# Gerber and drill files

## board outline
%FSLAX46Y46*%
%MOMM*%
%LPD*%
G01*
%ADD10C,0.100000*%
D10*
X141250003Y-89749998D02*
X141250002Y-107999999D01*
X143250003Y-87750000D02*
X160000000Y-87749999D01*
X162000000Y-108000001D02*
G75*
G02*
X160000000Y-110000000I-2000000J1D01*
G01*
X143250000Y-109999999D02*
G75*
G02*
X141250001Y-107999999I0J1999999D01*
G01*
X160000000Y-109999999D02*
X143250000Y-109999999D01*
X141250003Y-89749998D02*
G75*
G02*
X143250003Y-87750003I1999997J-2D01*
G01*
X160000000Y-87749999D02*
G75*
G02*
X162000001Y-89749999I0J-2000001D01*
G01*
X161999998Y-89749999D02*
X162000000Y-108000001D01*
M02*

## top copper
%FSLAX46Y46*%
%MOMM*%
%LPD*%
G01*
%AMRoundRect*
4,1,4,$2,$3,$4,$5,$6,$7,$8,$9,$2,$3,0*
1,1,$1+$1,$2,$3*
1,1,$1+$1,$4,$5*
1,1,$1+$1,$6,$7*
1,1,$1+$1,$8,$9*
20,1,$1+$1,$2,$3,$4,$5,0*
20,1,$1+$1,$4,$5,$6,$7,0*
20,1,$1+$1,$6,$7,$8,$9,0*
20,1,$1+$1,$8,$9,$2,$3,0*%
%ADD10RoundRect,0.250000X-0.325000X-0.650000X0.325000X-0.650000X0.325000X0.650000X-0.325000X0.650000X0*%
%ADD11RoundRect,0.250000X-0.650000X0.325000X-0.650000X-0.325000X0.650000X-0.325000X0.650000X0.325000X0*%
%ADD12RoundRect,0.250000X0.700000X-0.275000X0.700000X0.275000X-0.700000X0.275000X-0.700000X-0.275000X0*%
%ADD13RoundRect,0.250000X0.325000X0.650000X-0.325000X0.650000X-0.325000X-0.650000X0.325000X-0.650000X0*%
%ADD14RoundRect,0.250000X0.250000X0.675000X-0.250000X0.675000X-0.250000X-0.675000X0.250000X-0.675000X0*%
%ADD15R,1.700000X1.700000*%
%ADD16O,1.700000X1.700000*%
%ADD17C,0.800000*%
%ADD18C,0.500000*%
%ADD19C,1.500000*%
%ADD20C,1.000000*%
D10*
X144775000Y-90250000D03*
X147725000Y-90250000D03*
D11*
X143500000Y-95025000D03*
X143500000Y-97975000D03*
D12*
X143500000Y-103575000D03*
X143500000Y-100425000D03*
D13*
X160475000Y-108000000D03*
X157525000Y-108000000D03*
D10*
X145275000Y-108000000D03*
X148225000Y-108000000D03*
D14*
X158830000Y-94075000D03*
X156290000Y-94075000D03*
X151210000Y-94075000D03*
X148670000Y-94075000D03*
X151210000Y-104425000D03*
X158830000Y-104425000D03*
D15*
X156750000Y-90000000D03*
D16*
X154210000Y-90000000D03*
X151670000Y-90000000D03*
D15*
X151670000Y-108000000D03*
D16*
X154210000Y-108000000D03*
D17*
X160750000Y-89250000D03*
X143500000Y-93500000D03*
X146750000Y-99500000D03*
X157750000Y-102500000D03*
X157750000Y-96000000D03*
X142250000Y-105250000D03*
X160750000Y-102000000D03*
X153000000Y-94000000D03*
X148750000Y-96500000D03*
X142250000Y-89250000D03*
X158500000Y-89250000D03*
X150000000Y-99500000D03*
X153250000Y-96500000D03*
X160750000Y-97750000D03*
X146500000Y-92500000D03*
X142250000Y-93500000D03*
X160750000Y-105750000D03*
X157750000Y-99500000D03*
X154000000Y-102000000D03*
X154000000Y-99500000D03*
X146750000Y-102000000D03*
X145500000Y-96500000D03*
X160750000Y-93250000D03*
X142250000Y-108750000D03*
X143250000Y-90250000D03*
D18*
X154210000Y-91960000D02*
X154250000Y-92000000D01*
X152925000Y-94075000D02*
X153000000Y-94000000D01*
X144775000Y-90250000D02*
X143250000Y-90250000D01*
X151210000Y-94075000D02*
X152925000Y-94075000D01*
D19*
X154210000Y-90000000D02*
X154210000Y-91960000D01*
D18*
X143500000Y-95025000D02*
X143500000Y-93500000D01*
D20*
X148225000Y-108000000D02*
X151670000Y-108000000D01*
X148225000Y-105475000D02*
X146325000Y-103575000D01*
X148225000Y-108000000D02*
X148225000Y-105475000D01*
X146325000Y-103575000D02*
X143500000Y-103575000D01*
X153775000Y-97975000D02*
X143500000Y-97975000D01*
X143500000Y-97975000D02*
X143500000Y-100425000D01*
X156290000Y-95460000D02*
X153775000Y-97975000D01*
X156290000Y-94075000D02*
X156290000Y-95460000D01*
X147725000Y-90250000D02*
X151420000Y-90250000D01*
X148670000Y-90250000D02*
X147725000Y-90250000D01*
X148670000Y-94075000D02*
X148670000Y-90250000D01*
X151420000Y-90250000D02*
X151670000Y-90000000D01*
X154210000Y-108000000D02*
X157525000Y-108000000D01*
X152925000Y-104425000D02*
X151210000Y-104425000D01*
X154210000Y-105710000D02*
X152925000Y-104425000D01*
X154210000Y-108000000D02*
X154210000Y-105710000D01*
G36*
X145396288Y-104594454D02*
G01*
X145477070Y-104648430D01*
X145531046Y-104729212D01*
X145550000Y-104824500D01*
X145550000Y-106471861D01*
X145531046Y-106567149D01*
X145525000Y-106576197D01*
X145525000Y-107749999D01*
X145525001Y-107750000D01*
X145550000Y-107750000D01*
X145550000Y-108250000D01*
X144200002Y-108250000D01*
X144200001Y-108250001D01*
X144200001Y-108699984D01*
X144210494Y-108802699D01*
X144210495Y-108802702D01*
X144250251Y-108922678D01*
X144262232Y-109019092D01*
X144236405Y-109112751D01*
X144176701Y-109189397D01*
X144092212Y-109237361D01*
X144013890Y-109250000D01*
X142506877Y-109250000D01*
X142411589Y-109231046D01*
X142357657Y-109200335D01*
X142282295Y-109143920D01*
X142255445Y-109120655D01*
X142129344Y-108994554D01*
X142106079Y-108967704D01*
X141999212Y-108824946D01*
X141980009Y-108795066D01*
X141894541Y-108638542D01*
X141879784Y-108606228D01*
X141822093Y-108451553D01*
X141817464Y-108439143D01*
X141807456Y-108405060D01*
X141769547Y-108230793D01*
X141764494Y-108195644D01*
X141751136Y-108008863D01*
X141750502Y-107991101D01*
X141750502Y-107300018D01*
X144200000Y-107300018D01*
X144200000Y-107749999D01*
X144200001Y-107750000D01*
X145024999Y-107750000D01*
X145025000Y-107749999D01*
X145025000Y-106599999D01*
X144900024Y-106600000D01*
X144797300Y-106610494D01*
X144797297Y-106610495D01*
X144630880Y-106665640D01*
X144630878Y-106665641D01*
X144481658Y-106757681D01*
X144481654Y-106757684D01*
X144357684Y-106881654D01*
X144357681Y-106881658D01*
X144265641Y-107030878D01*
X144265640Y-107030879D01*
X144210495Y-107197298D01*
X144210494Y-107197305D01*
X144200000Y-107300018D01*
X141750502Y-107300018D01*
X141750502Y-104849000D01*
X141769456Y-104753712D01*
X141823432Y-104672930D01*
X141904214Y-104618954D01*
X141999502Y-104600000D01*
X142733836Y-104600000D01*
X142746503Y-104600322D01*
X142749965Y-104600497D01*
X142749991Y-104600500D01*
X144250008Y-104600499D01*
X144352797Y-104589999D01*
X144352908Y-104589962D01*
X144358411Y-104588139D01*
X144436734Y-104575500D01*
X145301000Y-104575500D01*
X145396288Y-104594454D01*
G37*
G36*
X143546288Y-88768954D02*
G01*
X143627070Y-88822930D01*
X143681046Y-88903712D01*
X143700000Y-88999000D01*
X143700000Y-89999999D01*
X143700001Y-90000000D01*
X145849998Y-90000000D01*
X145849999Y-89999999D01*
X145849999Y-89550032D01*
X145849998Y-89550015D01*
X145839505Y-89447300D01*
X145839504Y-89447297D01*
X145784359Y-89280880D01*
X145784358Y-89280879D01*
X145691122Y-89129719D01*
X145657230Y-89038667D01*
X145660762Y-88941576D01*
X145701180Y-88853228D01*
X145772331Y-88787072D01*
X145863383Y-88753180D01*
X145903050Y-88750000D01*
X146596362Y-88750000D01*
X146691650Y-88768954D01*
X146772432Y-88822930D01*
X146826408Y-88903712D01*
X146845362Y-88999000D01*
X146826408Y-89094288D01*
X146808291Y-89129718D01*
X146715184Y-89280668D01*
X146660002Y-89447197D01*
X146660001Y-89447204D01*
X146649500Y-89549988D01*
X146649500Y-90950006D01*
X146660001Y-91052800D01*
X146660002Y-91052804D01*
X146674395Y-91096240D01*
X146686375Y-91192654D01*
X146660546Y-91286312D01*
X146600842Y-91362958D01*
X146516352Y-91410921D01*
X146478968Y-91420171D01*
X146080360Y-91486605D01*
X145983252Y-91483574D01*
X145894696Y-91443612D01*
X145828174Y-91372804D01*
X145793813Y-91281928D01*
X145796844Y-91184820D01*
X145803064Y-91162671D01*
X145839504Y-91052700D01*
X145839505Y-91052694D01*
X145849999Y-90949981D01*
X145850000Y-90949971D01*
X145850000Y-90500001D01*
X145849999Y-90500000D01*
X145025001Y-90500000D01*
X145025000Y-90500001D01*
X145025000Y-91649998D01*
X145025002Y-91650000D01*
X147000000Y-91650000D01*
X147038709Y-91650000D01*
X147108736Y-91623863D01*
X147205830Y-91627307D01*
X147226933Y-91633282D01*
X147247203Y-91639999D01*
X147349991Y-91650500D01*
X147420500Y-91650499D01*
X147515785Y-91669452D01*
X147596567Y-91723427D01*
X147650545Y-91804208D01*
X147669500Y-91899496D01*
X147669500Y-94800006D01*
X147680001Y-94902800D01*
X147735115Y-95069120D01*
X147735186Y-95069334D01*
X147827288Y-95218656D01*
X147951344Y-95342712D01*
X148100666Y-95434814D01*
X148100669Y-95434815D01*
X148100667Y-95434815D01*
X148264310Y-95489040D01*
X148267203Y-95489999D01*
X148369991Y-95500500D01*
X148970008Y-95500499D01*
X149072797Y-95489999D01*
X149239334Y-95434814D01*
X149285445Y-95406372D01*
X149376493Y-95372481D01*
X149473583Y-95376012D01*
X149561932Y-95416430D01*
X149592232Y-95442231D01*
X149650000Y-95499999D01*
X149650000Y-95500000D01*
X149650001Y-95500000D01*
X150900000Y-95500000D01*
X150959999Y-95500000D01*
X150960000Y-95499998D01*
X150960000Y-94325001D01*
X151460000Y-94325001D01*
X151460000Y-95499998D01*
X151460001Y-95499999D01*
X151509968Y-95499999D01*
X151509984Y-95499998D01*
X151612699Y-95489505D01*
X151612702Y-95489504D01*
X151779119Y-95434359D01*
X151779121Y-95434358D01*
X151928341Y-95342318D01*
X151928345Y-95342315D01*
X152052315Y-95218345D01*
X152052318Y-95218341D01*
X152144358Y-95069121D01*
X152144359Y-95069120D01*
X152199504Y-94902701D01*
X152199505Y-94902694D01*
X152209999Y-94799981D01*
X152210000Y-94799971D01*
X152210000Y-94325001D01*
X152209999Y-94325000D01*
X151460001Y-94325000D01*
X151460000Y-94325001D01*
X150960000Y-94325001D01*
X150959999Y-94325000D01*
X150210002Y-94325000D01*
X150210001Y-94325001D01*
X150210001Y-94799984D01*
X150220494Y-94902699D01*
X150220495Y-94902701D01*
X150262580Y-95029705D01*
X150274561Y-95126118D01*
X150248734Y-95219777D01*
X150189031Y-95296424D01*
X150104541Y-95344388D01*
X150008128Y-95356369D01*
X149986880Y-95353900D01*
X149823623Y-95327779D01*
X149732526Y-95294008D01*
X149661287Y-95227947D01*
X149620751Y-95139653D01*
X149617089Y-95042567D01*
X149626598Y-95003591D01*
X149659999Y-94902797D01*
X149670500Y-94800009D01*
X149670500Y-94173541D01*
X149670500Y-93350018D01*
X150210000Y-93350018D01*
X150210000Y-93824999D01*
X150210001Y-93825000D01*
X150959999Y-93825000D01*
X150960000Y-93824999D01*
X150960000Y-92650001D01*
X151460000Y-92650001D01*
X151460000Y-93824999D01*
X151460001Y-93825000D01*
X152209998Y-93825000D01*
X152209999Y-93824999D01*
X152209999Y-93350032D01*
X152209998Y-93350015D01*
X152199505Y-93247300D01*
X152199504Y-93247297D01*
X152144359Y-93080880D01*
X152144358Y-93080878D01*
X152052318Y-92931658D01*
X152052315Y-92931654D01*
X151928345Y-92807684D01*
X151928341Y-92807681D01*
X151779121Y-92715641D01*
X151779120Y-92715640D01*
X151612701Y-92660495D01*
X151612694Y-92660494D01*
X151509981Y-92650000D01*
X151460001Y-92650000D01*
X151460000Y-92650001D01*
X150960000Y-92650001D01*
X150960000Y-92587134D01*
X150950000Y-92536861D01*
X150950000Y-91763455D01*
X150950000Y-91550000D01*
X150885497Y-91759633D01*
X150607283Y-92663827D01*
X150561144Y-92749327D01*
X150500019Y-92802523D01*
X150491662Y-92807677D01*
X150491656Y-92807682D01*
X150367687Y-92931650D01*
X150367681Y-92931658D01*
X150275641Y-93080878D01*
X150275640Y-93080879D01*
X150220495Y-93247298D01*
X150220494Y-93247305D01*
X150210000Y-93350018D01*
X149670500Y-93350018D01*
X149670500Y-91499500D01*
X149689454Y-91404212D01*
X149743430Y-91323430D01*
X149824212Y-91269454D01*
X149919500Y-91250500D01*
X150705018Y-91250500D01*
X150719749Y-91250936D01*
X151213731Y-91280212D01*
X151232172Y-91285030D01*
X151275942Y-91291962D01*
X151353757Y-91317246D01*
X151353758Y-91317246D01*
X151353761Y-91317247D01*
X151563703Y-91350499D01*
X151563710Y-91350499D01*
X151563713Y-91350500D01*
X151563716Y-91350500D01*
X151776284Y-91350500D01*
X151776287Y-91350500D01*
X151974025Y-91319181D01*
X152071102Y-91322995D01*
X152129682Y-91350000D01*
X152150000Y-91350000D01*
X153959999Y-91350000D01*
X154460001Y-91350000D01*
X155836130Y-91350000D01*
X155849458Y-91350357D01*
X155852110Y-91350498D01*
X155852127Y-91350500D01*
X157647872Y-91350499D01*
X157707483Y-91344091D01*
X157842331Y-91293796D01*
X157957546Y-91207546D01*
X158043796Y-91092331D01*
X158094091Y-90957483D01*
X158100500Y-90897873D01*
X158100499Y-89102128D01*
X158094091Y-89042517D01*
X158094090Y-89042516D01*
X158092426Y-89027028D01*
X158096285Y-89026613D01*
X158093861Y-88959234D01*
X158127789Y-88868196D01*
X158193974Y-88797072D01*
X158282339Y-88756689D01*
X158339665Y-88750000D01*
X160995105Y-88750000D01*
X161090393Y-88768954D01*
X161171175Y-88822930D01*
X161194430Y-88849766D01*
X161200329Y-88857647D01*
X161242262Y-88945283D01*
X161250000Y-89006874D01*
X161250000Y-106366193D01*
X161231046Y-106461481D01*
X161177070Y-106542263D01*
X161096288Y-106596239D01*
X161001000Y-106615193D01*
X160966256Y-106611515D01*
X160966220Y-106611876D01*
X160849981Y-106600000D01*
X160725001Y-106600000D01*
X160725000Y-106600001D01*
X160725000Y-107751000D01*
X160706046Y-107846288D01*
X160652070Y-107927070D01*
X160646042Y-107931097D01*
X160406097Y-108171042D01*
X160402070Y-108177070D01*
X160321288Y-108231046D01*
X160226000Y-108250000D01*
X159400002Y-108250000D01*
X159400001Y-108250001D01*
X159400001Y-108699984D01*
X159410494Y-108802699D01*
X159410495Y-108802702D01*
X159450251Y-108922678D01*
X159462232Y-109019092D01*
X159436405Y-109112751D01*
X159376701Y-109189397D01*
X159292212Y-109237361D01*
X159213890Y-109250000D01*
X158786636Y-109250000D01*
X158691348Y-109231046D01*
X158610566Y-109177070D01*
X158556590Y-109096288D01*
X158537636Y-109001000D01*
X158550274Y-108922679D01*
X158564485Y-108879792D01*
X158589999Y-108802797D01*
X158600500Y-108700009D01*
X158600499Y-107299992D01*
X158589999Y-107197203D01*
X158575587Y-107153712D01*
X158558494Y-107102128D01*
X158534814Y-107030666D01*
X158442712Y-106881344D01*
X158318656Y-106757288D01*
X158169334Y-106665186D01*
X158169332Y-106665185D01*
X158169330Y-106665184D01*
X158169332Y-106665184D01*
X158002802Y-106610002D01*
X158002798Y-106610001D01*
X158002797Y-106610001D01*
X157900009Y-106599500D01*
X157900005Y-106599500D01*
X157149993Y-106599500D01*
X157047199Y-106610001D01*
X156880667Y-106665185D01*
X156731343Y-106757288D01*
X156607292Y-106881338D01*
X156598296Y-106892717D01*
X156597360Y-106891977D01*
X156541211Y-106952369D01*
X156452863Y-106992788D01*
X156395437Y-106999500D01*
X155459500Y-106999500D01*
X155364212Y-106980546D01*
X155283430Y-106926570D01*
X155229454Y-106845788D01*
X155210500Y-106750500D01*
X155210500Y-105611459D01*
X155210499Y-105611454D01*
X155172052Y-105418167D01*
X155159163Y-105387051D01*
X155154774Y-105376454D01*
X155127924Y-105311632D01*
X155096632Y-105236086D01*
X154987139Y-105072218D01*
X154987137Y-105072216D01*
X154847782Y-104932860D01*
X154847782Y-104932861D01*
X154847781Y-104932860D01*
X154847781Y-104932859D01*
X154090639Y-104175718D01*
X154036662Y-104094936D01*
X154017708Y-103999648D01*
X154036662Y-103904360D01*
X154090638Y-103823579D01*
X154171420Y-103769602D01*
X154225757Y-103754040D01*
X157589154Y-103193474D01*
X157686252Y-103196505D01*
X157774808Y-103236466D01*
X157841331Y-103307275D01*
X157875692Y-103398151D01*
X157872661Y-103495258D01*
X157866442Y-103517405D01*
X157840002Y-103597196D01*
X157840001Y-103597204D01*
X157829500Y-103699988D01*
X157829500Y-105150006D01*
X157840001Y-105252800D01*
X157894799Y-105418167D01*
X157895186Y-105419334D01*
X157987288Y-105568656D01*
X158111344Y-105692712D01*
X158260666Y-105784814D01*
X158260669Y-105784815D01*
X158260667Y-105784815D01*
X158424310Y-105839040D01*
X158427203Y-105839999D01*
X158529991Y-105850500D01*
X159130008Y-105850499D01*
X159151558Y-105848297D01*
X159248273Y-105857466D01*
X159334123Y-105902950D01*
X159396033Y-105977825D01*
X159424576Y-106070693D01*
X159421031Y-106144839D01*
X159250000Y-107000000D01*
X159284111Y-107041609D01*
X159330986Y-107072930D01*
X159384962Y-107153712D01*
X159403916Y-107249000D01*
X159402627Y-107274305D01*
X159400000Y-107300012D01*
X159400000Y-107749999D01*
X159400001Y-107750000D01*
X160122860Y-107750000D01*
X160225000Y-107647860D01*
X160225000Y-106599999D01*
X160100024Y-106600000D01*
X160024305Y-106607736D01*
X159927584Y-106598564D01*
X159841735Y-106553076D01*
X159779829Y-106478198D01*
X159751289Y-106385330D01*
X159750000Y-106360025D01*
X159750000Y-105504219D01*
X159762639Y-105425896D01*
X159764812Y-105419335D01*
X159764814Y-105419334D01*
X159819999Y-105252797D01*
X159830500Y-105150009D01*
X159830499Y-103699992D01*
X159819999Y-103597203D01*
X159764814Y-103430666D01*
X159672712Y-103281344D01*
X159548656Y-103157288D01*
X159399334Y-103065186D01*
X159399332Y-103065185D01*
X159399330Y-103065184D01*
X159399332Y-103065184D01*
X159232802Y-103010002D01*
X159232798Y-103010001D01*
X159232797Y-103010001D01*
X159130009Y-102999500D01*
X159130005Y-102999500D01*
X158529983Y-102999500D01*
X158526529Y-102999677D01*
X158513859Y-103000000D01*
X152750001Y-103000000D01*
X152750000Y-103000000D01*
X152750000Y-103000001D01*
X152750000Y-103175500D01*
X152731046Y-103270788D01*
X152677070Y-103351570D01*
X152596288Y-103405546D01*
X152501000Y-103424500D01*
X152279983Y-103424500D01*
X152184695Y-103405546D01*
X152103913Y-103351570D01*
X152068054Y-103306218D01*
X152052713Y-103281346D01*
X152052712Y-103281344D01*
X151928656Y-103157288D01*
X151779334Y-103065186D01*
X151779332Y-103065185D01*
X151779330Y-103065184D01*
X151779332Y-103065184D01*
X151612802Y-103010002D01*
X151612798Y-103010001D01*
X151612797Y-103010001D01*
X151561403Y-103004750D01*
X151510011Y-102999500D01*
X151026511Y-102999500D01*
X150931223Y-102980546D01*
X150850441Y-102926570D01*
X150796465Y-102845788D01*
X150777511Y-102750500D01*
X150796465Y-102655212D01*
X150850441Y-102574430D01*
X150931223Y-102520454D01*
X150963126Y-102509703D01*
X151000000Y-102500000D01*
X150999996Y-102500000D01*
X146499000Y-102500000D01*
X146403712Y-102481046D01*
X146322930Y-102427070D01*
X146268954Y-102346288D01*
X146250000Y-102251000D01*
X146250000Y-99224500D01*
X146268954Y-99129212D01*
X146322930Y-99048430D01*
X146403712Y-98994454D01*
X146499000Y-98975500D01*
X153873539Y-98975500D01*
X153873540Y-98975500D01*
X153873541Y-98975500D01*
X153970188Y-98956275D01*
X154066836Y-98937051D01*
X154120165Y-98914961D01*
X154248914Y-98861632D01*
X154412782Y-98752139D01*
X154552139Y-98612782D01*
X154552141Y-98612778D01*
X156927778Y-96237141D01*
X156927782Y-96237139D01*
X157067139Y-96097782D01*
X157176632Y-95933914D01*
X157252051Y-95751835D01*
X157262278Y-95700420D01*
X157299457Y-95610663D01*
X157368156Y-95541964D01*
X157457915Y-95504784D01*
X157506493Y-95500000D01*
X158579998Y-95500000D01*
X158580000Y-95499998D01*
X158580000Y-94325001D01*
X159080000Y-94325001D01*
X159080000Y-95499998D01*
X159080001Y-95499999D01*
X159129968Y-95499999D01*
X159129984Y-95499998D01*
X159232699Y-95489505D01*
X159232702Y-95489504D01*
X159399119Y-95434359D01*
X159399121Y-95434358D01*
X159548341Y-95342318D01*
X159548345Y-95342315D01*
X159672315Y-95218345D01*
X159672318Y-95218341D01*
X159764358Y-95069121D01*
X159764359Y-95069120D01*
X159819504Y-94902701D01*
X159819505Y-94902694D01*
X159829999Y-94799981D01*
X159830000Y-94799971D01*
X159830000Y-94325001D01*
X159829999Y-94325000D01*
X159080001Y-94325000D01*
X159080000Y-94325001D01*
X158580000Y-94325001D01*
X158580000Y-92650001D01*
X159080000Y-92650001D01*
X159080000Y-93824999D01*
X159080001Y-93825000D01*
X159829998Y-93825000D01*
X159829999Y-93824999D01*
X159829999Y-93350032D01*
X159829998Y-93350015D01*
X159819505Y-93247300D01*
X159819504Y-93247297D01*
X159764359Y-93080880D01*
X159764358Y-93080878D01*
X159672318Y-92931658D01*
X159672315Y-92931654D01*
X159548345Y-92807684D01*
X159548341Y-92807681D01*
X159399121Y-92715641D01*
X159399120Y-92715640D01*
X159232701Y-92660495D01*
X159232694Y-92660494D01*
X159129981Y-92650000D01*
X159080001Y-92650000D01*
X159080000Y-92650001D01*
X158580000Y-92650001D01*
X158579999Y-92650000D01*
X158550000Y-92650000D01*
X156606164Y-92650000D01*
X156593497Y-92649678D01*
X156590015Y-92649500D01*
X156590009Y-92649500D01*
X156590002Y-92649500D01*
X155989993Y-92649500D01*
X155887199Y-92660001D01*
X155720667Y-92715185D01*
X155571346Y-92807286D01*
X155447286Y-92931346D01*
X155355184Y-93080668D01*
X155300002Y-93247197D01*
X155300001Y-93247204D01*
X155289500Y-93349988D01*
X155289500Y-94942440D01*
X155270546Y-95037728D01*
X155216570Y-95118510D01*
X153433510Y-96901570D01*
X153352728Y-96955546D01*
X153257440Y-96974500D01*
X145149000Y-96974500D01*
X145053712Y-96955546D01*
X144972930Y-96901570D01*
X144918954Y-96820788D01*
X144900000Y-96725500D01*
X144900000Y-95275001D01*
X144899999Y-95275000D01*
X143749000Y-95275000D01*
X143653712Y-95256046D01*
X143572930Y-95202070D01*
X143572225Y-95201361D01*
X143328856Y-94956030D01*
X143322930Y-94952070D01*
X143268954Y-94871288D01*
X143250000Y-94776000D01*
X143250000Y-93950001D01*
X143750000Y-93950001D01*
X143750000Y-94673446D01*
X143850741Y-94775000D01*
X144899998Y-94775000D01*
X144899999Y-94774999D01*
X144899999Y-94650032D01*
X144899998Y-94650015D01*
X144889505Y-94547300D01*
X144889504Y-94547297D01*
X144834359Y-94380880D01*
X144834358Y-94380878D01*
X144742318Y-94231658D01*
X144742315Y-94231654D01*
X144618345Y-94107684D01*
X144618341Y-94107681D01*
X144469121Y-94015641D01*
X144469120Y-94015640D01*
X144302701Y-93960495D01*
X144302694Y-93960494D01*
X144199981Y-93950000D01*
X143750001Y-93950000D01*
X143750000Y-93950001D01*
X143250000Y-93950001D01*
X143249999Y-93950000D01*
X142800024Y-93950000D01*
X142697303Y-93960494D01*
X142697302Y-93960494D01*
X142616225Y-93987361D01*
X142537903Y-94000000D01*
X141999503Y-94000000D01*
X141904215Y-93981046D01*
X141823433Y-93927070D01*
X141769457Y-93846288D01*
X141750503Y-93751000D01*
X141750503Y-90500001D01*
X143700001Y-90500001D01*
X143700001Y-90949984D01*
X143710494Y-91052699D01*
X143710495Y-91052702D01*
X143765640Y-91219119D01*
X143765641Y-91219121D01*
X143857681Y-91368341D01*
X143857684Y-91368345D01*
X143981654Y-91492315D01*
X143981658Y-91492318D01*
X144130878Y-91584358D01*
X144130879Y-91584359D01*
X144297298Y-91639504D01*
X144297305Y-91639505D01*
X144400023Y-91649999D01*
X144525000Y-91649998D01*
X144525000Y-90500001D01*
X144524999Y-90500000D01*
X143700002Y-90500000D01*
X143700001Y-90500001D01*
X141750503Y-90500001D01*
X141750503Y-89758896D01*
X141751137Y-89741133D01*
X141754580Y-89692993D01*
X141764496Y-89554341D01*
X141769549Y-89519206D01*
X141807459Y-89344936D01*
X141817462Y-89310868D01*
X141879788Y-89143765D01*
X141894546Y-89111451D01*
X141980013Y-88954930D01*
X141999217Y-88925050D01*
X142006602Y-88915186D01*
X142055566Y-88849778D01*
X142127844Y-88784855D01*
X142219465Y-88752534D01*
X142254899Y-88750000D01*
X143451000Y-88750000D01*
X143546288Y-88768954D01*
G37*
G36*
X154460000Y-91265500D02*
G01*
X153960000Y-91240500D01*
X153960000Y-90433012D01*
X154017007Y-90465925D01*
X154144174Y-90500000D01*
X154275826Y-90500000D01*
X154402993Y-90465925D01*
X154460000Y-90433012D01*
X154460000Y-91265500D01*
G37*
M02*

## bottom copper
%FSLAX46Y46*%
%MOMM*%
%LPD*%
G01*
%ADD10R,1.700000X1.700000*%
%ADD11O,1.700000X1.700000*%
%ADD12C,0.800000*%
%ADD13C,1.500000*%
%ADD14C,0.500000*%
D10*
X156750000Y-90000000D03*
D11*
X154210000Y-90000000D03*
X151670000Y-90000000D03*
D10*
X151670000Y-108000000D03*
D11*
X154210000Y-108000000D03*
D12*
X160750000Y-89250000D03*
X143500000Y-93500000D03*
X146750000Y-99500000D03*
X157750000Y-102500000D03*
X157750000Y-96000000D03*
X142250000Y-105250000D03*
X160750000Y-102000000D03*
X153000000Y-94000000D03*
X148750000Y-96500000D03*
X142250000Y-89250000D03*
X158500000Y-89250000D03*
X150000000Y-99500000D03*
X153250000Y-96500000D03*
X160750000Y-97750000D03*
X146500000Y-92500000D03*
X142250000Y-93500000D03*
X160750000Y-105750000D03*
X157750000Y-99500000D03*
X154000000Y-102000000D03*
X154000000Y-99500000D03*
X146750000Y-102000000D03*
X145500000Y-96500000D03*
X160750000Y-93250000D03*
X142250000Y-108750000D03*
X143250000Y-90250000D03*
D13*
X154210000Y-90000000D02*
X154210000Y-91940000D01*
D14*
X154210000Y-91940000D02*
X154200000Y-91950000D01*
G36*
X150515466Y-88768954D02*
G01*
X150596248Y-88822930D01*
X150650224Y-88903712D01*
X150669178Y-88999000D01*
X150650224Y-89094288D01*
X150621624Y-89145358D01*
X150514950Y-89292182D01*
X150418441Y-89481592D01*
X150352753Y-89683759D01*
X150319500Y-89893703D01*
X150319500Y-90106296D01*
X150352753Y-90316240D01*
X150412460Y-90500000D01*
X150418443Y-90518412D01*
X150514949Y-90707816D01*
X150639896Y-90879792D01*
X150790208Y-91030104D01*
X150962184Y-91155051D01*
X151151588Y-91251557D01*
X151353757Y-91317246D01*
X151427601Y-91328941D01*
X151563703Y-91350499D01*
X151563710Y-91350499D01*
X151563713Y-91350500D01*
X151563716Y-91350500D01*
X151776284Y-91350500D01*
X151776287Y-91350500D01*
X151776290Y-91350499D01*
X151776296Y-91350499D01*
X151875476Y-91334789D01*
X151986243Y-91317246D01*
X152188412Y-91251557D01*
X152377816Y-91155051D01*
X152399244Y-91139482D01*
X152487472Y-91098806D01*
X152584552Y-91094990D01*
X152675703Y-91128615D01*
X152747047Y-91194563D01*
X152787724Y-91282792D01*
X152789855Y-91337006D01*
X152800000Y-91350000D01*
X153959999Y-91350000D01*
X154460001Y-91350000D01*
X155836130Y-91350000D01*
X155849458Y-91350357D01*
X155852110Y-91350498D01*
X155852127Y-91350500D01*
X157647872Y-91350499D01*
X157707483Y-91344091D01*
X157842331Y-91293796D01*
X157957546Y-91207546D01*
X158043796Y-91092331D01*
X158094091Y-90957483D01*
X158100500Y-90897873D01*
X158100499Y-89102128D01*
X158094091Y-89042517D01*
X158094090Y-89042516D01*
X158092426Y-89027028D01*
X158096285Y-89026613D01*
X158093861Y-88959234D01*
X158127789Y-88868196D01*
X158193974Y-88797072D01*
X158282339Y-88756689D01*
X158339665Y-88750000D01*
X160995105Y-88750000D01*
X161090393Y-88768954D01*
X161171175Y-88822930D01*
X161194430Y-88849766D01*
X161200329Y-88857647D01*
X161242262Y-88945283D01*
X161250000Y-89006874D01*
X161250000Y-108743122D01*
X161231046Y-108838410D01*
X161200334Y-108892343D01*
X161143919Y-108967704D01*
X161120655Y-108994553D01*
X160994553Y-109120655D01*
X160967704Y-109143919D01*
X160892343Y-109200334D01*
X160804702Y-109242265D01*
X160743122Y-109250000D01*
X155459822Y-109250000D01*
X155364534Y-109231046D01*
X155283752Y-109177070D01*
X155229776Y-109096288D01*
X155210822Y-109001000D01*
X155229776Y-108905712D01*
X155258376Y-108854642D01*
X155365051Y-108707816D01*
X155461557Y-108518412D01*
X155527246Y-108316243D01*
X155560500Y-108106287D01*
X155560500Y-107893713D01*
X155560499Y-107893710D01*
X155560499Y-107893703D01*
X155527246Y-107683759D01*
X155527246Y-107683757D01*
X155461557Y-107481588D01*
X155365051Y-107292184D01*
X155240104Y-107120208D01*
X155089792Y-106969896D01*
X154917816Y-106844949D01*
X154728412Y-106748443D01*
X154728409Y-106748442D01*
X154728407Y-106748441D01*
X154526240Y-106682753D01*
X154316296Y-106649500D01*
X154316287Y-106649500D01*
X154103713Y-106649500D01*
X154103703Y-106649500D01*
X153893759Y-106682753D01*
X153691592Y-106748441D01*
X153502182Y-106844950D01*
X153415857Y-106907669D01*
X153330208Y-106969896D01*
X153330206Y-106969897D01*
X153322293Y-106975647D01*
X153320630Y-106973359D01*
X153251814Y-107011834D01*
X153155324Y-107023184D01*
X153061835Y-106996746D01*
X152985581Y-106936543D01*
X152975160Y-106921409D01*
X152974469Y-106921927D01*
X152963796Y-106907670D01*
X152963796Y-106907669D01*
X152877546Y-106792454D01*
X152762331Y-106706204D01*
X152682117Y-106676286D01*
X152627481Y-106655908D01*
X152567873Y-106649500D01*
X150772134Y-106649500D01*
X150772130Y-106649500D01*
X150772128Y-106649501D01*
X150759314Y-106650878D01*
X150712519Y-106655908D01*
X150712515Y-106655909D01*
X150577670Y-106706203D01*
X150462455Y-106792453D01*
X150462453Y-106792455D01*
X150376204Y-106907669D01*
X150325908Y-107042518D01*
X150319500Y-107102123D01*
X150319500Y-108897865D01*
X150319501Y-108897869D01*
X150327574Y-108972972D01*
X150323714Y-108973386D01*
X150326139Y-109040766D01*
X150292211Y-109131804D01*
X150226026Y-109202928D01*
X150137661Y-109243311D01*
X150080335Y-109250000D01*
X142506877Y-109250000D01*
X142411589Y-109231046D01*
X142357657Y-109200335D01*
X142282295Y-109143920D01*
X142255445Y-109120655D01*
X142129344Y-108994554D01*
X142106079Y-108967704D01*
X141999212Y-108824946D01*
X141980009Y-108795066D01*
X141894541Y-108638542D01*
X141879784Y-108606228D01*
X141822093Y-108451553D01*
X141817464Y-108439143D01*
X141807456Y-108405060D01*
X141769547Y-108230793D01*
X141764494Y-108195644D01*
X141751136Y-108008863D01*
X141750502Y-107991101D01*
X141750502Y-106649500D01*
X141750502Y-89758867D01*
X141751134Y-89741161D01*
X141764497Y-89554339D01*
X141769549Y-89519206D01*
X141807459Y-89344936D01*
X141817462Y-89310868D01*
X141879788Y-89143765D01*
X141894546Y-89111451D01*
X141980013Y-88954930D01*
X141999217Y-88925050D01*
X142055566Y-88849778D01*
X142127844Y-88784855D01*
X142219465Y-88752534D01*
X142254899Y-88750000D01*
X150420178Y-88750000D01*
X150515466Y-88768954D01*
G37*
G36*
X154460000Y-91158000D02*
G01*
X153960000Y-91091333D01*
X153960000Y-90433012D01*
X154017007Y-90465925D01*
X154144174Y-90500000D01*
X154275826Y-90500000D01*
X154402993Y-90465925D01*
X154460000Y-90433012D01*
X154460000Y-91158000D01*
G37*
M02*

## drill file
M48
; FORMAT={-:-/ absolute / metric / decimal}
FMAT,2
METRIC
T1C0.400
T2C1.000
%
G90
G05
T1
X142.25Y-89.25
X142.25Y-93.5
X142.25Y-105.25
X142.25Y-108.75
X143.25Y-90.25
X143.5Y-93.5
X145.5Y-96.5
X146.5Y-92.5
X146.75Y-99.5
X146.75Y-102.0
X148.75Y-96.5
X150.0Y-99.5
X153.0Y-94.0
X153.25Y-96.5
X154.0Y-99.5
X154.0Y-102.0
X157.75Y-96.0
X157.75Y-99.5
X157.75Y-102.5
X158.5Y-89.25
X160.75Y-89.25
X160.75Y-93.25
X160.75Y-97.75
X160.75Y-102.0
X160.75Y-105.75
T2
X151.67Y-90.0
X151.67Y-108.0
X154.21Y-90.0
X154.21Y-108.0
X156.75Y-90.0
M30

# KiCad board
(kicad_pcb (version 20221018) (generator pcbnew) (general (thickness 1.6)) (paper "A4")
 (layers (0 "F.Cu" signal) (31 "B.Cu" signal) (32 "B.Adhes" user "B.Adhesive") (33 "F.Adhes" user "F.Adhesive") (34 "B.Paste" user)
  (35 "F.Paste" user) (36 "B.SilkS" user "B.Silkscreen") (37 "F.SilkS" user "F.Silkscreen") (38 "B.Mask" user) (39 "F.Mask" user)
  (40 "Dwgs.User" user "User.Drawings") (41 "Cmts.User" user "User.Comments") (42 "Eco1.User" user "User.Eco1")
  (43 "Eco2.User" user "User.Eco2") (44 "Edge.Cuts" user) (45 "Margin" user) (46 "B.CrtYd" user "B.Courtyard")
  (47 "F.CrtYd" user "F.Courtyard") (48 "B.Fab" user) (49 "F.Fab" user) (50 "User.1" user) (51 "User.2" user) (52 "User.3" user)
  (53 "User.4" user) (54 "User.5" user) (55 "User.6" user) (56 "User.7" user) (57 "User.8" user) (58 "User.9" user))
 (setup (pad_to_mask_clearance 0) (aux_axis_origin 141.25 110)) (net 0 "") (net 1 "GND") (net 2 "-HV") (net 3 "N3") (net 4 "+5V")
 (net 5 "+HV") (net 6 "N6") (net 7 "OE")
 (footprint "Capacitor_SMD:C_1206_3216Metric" (layer "F.Cu") (at 146.25 90.25)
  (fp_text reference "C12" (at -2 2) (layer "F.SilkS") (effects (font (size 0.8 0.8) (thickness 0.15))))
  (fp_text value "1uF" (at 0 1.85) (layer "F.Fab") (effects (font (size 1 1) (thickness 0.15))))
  (pad "1" smd roundrect (at -1.475 0) (size 1.15 1.8) (layers "F.Cu" "F.Paste" "F.Mask") (roundrect_rratio 0.2173913043) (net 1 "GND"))
  (pad "2" smd roundrect (at 1.475 0) (size 1.15 1.8) (layers "F.Cu" "F.Paste" "F.Mask") (roundrect_rratio 0.2173913043) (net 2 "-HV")))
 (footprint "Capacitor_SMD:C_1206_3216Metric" (layer "F.Cu") (at 143.5 96.5 -90)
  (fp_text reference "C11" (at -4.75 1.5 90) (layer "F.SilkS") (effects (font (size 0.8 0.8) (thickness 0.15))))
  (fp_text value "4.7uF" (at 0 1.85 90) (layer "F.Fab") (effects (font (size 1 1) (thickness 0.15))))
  (pad "1" smd roundrect (at -1.475 0 270) (size 1.15 1.8) (layers "F.Cu" "F.Paste" "F.Mask") (roundrect_rratio 0.2173913043) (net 1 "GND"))
  (pad "2" smd roundrect (at 1.475 0 270) (size 1.15 1.8) (layers "F.Cu" "F.Paste" "F.Mask") (roundrect_rratio 0.2173913043) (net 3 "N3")))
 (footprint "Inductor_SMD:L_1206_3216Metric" (layer "F.Cu") (at 143.5 102 90)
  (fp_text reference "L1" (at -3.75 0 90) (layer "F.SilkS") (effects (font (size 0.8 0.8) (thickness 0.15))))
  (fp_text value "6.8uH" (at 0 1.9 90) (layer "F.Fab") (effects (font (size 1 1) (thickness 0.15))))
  (pad "1" smd roundrect (at -1.575 0 90) (size 1.05 1.9) (layers "F.Cu" "F.Paste" "F.Mask") (roundrect_rratio 0.2380952381) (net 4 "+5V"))
  (pad "2" smd roundrect (at 1.575 0 90) (size 1.05 1.9) (layers "F.Cu" "F.Paste" "F.Mask") (roundrect_rratio 0.2380952381) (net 3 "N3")))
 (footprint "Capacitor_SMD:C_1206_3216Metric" (layer "F.Cu") (at 159 108 180)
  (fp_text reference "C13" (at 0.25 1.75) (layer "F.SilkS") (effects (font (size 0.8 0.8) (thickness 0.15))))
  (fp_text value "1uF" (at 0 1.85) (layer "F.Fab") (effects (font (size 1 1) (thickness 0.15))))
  (pad "1" smd roundrect (at -1.475 0 180) (size 1.15 1.8) (layers "F.Cu" "F.Paste" "F.Mask") (roundrect_rratio 0.2173913043) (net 1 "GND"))
  (pad "2" smd roundrect (at 1.475 0 180) (size 1.15 1.8) (layers "F.Cu" "F.Paste" "F.Mask") (roundrect_rratio 0.2173913043) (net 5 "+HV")))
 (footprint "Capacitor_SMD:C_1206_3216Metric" (layer "F.Cu") (at 146.75 108)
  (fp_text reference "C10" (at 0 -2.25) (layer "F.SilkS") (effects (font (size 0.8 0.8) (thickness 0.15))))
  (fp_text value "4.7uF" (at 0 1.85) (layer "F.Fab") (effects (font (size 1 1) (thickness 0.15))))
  (pad "1" smd roundrect (at -1.475 0) (size 1.15 1.8) (layers "F.Cu" "F.Paste" "F.Mask") (roundrect_rratio 0.2173913043) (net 1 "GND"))
  (pad "2" smd roundrect (at 1.475 0) (size 1.15 1.8) (layers "F.Cu" "F.Paste" "F.Mask") (roundrect_rratio 0.2173913043) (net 4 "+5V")))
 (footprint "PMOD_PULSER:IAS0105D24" (layer "F.Cu") (at 153.75 99.25 180)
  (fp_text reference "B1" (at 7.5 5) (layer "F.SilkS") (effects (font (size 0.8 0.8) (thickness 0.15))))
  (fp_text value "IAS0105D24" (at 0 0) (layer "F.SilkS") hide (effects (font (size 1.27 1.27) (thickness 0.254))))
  (pad "1" smd roundrect (at -5.08 5.175 180) (size 1 1.85) (layers "F.Cu" "F.Paste" "F.Mask") (roundrect_rratio 0.25) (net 1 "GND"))
  (pad "2" smd roundrect (at -2.54 5.175 180) (size 1 1.85) (layers "F.Cu" "F.Paste" "F.Mask") (roundrect_rratio 0.25) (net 3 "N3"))
  (pad "4" smd roundrect (at 2.54 5.175 180) (size 1 1.85) (layers "F.Cu" "F.Paste" "F.Mask") (roundrect_rratio 0.25) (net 1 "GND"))
  (pad "5" smd roundrect (at 5.08 5.175 180) (size 1 1.85) (layers "F.Cu" "F.Paste" "F.Mask") (roundrect_rratio 0.25) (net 2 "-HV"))
  (pad "7" smd roundrect (at 2.54 -5.175 180) (size 1 1.85) (layers "F.Cu" "F.Paste" "F.Mask") (roundrect_rratio 0.25) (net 5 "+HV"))
  (pad "10" smd roundrect (at -5.08 -5.175 180) (size 1 1.85) (layers "F.Cu" "F.Paste" "F.Mask") (roundrect_rratio 0.25) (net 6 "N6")))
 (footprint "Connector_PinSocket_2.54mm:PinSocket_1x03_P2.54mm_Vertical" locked (layer "B.Cu") (at 156.75 90 90)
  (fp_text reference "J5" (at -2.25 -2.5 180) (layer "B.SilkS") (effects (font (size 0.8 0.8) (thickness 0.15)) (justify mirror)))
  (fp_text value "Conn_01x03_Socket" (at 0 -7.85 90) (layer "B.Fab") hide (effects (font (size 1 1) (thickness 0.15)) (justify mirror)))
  (pad "1" thru_hole rect locked (at 0 0 90) (size 1.7 1.7) (drill 1) (layers "*.Cu" "*.Mask") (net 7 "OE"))
  (pad "2" thru_hole oval locked (at 0 -2.54 90) (size 1.7 1.7) (drill 1) (layers "*.Cu" "*.Mask") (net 1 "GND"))
  (pad "3" thru_hole oval locked (at 0 -5.08 90) (size 1.7 1.7) (drill 1) (layers "*.Cu" "*.Mask") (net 2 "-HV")))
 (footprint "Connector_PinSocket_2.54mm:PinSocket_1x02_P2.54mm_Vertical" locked (layer "B.Cu") (at 151.67 108 -90)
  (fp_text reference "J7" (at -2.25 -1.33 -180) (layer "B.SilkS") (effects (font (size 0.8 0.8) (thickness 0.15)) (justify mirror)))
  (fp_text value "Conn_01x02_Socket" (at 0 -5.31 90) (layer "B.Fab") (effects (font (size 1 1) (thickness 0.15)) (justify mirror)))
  (pad "1" thru_hole rect locked (at 0 0 270) (size 1.7 1.7) (drill 1) (layers "*.Cu" "*.Mask") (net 4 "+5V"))
  (pad "2" thru_hole oval locked (at 0 -2.54 270) (size 1.7 1.7) (drill 1) (layers "*.Cu" "*.Mask") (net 5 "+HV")))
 (gr_line (start 141.250003 89.749998) (end 141.250002 107.999999) (stroke (width 0.1) (type default)) (layer "Edge.Cuts"))
 (gr_line (start 143.250003 87.75) (end 160 87.749999) (stroke (width 0.1) (type default)) (layer "Edge.Cuts"))
 (gr_arc (start 162 108.000001) (mid 161.414213 109.414213) (end 160 109.999999) (stroke (width 0.1) (type default)) (layer "Edge.Cuts"))
 (gr_arc (start 143.25 109.999999) (mid 141.835786 109.414213) (end 141.250002 107.999999) (stroke (width 0.1) (type default))
  (layer "Edge.Cuts"))
 (gr_line (start 160 109.999999) (end 143.25 109.999999) (stroke (width 0.1) (type default)) (layer "Edge.Cuts"))
 (gr_arc (start 141.250003 89.749998) (mid 141.83579 88.335786) (end 143.250003 87.75) (stroke (width 0.1) (type default))
  (layer "Edge.Cuts"))
 (gr_arc (start 160 87.749999) (mid 161.414214 88.335785) (end 161.999998 89.749999) (stroke (width 0.1) (type default)) (layer "Edge.Cuts"))
 (gr_line (start 161.999998 89.749999) (end 162 108.000001) (stroke (width 0.1) (type default)) (layer "Edge.Cuts"))
 (segment (start 154.21 91.96) (end 154.25 92) (width 0.5) (layer "F.Cu") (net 1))
 (segment (start 152.925 94.075) (end 153 94) (width 0.5) (layer "F.Cu") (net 1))
 (segment (start 144.775 90.25) (end 143.25 90.25) (width 0.5) (layer "F.Cu") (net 1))
 (segment (start 151.21 94.075) (end 152.925 94.075) (width 0.5) (layer "F.Cu") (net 1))
 (segment (start 154.21 90) (end 154.21 91.96) (width 1.5) (layer "F.Cu") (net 1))
 (segment (start 143.5 95.025) (end 143.5 93.5) (width 0.5) (layer "F.Cu") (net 1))
 (via (at 160.75 89.25) (size 0.8) (drill 0.4) (layers "F.Cu" "B.Cu") (free) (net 1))
 (via (at 143.5 93.5) (size 0.8) (drill 0.4) (layers "F.Cu" "B.Cu") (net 1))
 (via (at 146.75 99.5) (size 0.8) (drill 0.4) (layers "F.Cu" "B.Cu") (free) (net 1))
 (via (at 157.75 102.5) (size 0.8) (drill 0.4) (layers "F.Cu" "B.Cu") (free) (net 1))
 (via (at 157.75 96) (size 0.8) (drill 0.4) (layers "F.Cu" "B.Cu") (free) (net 1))
 (via (at 142.25 105.25) (size 0.8) (drill 0.4) (layers "F.Cu" "B.Cu") (free) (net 1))
 (via (at 160.75 102) (size 0.8) (drill 0.4) (layers "F.Cu" "B.Cu") (free) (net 1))
 (via (at 153 94) (size 0.8) (drill 0.4) (layers "F.Cu" "B.Cu") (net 1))
 (via (at 148.75 96.5) (size 0.8) (drill 0.4) (layers "F.Cu" "B.Cu") (free) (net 1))
 (via (at 142.25 89.25) (size 0.8) (drill 0.4) (layers "F.Cu" "B.Cu") (free) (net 1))
 (via (at 158.5 89.25) (size 0.8) (drill 0.4) (layers "F.Cu" "B.Cu") (free) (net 1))
 (via (at 150 99.5) (size 0.8) (drill 0.4) (layers "F.Cu" "B.Cu") (free) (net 1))
 (via (at 153.25 96.5) (size 0.8) (drill 0.4) (layers "F.Cu" "B.Cu") (free) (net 1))
 (via (at 160.75 97.75) (size 0.8) (drill 0.4) (layers "F.Cu" "B.Cu") (free) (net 1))
 (via (at 146.5 92.5) (size 0.8) (drill 0.4) (layers "F.Cu" "B.Cu") (free) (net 1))
 (via (at 142.25 93.5) (size 0.8) (drill 0.4) (layers "F.Cu" "B.Cu") (free) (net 1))
 (via (at 160.75 105.75) (size 0.8) (drill 0.4) (layers "F.Cu" "B.Cu") (free) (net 1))
 (via (at 157.75 99.5) (size 0.8) (drill 0.4) (layers "F.Cu" "B.Cu") (free) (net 1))
 (via (at 154 102) (size 0.8) (drill 0.4) (layers "F.Cu" "B.Cu") (free) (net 1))
 (via (at 154 99.5) (size 0.8) (drill 0.4) (layers "F.Cu" "B.Cu") (free) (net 1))
 (via (at 146.75 102) (size 0.8) (drill 0.4) (layers "F.Cu" "B.Cu") (free) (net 1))
 (via (at 145.5 96.5) (size 0.8) (drill 0.4) (layers "F.Cu" "B.Cu") (free) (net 1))
 (via (at 160.75 93.25) (size 0.8) (drill 0.4) (layers "F.Cu" "B.Cu") (free) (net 1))
 (via (at 142.25 108.75) (size 0.8) (drill 0.4) (layers "F.Cu" "B.Cu") (free) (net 1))
 (via (at 143.25 90.25) (size 0.8) (drill 0.4) (layers "F.Cu" "B.Cu") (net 1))
 (segment (start 154.21 90) (end 154.21 91.94) (width 1.5) (layer "B.Cu") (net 1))
 (segment (start 154.21 91.94) (end 154.2 91.95) (width 0.5) (layer "B.Cu") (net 1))
 (segment (start 148.225 108) (end 151.67 108) (width 1) (layer "F.Cu") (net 4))
 (segment (start 148.225 105.475) (end 146.325 103.575) (width 1) (layer "F.Cu") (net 4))
 (segment (start 148.225 108) (end 148.225 105.475) (width 1) (layer "F.Cu") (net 4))
 (segment (start 146.325 103.575) (end 143.5 103.575) (width 1) (layer "F.Cu") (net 4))
 (segment (start 153.775 97.975) (end 143.5 97.975) (width 1) (layer "F.Cu") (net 3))
 (segment (start 143.5 97.975) (end 143.5 100.425) (width 1) (layer "F.Cu") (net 3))
 (segment (start 156.29 95.46) (end 153.775 97.975) (width 1) (layer "F.Cu") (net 3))
 (segment (start 156.29 94.075) (end 156.29 95.46) (width 1) (layer "F.Cu") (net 3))
 (segment (start 147.725 90.25) (end 151.42 90.25) (width 1) (layer "F.Cu") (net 2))
 (segment (start 148.67 90.25) (end 147.725 90.25) (width 1) (layer "F.Cu") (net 2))
 (segment (start 148.67 94.075) (end 148.67 90.25) (width 1) (layer "F.Cu") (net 2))
 (segment (start 151.42 90.25) (end 151.67 90) (width 1) (layer "F.Cu") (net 2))
 (segment (start 154.21 108) (end 157.525 108) (width 1) (layer "F.Cu") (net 5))
 (segment (start 152.925 104.425) (end 151.21 104.425) (width 1) (layer "F.Cu") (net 5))
 (segment (start 154.21 105.71) (end 152.925 104.425) (width 1) (layer "F.Cu") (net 5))
 (segment (start 154.21 108) (end 154.21 105.71) (width 1) (layer "F.Cu") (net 5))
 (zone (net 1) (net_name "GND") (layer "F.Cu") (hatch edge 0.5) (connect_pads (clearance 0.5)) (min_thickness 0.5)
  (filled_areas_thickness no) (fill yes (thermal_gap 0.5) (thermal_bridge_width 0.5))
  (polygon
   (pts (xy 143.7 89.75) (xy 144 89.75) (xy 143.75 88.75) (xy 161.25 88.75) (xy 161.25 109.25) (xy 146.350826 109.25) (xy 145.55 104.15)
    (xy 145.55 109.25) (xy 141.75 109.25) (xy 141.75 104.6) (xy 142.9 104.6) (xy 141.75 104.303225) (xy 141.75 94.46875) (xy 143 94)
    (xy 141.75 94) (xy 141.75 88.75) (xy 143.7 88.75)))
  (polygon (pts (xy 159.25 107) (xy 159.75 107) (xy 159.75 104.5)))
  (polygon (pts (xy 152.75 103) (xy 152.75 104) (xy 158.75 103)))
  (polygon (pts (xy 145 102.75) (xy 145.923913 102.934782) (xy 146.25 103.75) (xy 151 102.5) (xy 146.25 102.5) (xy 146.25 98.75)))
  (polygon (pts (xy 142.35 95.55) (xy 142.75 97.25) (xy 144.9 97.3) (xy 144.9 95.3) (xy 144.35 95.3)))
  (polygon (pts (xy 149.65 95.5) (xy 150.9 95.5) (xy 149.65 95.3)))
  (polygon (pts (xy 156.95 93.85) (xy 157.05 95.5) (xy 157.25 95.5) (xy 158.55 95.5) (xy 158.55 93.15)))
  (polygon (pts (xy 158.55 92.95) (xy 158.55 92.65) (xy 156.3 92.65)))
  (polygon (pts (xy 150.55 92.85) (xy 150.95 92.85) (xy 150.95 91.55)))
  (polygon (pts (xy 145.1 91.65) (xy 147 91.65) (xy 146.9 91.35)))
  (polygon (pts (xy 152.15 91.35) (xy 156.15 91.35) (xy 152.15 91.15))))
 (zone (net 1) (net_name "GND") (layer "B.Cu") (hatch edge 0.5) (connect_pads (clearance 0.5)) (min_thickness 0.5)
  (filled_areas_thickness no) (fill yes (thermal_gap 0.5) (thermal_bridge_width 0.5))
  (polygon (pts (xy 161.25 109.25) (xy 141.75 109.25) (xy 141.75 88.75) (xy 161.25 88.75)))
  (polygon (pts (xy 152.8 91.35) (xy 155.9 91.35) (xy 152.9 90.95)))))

